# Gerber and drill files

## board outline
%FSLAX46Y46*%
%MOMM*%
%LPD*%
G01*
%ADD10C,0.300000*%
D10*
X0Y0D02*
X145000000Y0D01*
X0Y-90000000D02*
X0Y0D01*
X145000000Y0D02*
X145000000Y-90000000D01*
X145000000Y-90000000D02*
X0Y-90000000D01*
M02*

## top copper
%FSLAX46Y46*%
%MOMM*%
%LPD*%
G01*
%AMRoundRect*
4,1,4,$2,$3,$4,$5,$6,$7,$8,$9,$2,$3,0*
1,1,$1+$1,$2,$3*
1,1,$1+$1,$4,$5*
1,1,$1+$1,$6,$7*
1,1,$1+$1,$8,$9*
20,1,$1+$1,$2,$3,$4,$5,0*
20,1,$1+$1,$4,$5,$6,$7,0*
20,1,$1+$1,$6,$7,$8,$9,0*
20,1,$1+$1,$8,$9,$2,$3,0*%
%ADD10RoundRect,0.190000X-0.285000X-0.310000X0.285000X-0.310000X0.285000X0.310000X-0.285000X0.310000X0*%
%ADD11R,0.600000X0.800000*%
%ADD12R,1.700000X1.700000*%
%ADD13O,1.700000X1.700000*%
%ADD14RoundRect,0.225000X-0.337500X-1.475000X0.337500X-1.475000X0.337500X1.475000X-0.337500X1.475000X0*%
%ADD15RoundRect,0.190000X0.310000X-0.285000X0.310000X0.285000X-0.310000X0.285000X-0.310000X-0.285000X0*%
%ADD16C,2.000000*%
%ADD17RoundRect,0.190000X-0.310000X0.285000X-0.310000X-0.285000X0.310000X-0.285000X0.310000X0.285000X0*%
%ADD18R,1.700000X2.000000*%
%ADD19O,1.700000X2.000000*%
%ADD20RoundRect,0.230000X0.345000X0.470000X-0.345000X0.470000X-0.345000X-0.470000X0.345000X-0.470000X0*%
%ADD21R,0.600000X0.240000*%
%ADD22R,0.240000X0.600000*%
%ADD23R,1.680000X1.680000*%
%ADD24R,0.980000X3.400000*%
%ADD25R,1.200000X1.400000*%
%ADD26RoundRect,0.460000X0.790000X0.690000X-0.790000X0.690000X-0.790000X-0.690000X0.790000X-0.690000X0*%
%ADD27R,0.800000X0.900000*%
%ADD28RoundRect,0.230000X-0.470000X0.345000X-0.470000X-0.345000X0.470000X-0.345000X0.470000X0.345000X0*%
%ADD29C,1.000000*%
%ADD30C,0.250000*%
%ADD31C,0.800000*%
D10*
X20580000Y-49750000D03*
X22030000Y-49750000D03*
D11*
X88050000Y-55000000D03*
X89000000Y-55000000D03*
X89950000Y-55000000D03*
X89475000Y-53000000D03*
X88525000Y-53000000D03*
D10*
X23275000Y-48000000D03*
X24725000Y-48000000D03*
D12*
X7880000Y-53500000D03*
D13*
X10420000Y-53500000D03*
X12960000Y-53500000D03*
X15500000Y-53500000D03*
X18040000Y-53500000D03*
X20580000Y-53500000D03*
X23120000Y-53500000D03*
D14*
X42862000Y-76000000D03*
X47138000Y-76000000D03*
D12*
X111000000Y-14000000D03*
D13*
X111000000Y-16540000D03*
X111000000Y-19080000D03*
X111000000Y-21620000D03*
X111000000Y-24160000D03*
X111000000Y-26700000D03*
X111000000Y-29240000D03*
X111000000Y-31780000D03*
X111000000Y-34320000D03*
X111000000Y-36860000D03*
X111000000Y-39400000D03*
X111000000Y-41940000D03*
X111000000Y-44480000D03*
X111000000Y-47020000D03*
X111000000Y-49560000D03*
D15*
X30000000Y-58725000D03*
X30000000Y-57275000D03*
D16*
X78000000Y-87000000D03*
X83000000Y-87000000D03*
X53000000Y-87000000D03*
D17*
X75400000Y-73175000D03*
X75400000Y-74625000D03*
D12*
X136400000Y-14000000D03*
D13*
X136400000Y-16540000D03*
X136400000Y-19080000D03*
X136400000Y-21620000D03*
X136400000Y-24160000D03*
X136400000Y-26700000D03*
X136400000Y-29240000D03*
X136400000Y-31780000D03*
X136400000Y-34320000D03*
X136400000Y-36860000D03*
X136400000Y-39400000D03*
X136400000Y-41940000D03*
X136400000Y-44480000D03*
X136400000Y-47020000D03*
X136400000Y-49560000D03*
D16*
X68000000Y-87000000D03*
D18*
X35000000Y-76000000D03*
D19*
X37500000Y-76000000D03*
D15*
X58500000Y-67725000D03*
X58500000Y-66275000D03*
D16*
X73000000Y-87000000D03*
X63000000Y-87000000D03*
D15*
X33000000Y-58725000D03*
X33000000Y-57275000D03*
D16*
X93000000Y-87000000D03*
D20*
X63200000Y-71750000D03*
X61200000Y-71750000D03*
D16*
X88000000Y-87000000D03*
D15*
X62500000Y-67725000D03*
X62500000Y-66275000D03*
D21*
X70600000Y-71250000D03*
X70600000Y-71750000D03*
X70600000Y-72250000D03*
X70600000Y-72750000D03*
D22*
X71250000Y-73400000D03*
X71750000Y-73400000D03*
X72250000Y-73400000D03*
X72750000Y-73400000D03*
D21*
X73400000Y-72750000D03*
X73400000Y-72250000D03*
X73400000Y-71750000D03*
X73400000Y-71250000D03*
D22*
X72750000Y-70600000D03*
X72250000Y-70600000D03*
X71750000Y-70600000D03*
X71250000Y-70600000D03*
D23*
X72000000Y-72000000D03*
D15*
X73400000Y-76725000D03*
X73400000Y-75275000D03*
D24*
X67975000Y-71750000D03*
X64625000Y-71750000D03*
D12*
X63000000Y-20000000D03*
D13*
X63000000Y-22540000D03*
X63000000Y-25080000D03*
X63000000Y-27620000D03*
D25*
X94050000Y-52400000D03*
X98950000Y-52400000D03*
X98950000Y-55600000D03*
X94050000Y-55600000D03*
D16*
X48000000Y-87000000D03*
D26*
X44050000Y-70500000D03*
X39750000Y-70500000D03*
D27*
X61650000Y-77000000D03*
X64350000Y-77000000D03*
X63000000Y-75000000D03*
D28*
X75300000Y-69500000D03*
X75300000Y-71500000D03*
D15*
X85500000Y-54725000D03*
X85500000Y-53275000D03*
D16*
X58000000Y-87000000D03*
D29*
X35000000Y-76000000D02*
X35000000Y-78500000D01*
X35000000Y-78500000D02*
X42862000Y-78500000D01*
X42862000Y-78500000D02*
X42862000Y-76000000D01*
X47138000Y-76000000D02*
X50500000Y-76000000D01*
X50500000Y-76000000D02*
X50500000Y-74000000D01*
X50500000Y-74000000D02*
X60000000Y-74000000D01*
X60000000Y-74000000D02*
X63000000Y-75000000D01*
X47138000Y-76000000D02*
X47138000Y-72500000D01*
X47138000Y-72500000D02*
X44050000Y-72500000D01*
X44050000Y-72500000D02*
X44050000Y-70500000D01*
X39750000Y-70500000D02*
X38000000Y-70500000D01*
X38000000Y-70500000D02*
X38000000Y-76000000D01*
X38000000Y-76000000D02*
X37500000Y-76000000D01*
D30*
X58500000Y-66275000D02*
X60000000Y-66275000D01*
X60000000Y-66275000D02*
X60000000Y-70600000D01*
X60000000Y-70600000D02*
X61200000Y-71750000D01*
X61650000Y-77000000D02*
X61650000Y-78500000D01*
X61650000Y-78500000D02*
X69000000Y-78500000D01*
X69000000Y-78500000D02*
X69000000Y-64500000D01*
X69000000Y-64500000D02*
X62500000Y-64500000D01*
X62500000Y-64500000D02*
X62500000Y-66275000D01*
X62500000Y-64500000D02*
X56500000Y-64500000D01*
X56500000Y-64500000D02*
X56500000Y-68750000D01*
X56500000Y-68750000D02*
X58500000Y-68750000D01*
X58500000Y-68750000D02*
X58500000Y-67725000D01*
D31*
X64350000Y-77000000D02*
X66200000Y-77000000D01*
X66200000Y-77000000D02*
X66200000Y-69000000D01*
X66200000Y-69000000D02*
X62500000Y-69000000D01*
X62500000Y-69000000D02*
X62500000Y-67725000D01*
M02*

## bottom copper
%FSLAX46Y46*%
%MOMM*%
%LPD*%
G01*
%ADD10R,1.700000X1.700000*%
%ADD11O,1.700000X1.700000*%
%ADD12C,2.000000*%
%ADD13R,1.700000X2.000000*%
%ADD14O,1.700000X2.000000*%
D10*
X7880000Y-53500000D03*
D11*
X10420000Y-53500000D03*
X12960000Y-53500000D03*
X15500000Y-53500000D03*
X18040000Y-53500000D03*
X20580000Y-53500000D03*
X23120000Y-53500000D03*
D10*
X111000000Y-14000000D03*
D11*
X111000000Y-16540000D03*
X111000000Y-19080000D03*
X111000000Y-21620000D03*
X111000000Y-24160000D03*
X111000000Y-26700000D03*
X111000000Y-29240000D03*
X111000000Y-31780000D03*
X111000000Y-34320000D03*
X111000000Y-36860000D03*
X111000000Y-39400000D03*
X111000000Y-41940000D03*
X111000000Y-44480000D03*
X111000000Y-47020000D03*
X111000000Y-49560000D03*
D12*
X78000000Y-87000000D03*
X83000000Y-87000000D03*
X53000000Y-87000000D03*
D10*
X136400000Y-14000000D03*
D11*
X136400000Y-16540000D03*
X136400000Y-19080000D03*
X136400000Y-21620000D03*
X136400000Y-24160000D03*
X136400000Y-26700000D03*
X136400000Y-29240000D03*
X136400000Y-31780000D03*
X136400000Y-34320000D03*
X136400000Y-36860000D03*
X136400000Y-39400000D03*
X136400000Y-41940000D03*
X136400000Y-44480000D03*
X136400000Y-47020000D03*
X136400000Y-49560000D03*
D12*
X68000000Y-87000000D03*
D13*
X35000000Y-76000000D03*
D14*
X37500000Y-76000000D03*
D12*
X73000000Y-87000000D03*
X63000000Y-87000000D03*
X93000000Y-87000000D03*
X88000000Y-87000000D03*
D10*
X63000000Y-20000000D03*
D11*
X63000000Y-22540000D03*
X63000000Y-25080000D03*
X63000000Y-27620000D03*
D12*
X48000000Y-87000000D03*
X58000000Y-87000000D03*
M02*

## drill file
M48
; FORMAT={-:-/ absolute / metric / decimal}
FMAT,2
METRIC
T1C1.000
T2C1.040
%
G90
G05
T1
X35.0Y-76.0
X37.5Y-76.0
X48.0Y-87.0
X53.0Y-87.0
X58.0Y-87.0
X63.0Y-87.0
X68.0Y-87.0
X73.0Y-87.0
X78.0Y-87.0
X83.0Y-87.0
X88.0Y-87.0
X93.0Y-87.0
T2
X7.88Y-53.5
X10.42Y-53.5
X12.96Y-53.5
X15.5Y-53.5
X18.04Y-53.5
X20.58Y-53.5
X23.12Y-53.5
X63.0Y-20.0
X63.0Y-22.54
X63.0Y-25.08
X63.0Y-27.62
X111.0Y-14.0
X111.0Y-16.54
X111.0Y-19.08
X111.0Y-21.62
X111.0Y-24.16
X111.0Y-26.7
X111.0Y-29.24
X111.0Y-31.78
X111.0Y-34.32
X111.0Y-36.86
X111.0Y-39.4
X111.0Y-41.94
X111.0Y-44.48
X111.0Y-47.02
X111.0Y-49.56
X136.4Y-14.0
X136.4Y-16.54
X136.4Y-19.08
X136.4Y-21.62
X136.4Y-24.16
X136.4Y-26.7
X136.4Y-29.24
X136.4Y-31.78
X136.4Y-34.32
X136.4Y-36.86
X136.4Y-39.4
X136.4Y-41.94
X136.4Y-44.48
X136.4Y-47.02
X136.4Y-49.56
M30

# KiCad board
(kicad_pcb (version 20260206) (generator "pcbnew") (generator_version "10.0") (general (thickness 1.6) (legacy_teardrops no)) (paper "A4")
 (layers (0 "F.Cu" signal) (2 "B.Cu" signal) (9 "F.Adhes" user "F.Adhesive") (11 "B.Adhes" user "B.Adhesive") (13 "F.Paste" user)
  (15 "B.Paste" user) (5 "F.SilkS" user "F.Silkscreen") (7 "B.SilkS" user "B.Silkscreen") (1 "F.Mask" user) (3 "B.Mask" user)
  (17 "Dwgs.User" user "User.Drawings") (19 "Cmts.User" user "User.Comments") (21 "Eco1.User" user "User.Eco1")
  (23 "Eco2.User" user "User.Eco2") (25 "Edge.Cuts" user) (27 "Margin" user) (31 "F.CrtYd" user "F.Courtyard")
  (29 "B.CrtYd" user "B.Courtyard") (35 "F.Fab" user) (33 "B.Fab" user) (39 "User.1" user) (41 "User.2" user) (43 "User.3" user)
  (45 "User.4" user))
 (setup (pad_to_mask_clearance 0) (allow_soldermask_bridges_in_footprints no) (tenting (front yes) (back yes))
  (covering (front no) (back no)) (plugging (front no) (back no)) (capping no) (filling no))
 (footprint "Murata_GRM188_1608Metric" (layer "F.Cu") (at 21.305 49.75)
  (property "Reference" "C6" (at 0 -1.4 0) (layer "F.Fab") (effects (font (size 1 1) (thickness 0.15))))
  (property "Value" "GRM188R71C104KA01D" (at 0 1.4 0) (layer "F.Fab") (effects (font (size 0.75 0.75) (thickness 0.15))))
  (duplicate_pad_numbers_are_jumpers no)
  (pad "1" smd roundrect (at -0.725 0) (size 0.95 1) (layers "F.Cu" "F.Mask" "F.Paste") (roundrect_rratio 0.2) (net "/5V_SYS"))
  (pad "2" smd roundrect (at 0.725 0) (size 0.95 1) (layers "F.Cu" "F.Mask" "F.Paste") (roundrect_rratio 0.2) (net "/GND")))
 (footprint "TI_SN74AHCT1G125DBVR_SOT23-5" (layer "F.Cu") (at 89 54)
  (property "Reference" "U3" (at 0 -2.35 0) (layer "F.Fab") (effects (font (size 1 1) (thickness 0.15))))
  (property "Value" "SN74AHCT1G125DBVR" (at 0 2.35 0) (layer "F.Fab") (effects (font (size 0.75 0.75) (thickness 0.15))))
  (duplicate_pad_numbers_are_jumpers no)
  (pad "1" smd rect (at -0.95 1) (size 0.6 0.8) (layers "F.Cu" "F.Mask" "F.Paste") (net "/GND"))
  (pad "2" smd rect (at 0 1) (size 0.6 0.8) (layers "F.Cu" "F.Mask" "F.Paste") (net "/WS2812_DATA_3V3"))
  (pad "3" smd rect (at 0.95 1) (size 0.6 0.8) (layers "F.Cu" "F.Mask" "F.Paste") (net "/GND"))
  (pad "4" smd rect (at 0.475 -1) (size 0.6 0.8) (layers "F.Cu" "F.Mask" "F.Paste") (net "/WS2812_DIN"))
  (pad "5" smd rect (at -0.475 -1) (size 0.6 0.8) (layers "F.Cu" "F.Mask" "F.Paste") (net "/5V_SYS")))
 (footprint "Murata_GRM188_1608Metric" (layer "F.Cu") (at 24 48)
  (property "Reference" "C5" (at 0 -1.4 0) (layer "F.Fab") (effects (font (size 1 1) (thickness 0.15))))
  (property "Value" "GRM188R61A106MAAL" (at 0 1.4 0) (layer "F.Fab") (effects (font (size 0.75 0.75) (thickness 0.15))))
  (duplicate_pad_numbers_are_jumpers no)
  (pad "1" smd roundrect (at -0.725 0) (size 0.95 1) (layers "F.Cu" "F.Mask" "F.Paste") (roundrect_rratio 0.2) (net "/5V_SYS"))
  (pad "2" smd roundrect (at 0.725 0) (size 0.95 1) (layers "F.Cu" "F.Mask" "F.Paste") (roundrect_rratio 0.2) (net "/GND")))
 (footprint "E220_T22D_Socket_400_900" (layer "F.Cu") (at 5 52)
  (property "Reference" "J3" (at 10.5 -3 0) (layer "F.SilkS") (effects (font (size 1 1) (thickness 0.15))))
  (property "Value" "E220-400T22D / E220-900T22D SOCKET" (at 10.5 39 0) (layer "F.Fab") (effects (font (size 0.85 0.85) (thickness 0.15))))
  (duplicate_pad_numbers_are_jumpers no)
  (pad "1" thru_hole rect (at 2.88 1.5) (size 1.7 1.7) (drill 1.04) (layers "*.Cu" "*.Mask") (remove_unused_layers no) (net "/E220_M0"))
  (pad "2" thru_hole oval (at 5.42 1.5) (size 1.7 1.7) (drill 1.04) (layers "*.Cu" "*.Mask") (remove_unused_layers no) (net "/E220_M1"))
  (pad "3" thru_hole oval (at 7.96 1.5) (size 1.7 1.7) (drill 1.04) (layers "*.Cu" "*.Mask") (remove_unused_layers no) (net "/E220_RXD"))
  (pad "4" thru_hole oval (at 10.5 1.5) (size 1.7 1.7) (drill 1.04) (layers "*.Cu" "*.Mask") (remove_unused_layers no) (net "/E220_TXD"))
  (pad "5" thru_hole oval (at 13.04 1.5) (size 1.7 1.7) (drill 1.04) (layers "*.Cu" "*.Mask") (remove_unused_layers no) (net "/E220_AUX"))
  (pad "6" thru_hole oval (at 15.58 1.5) (size 1.7 1.7) (drill 1.04) (layers "*.Cu" "*.Mask") (remove_unused_layers no) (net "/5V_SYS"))
  (pad "7" thru_hole oval (at 18.12 1.5) (size 1.7 1.7) (drill 1.04) (layers "*.Cu" "*.Mask") (remove_unused_layers no) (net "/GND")))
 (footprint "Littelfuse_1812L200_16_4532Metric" (layer "F.Cu") (at 45 76)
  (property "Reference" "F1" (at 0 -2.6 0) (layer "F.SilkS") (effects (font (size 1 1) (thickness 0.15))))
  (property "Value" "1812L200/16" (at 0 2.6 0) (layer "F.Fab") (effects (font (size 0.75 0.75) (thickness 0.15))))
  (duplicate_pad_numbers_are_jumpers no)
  (pad "1" smd roundrect (at -2.138 0) (size 1.125 3.4) (layers "F.Cu" "F.Mask" "F.Paste") (roundrect_rratio 0.2) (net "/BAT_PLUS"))
  (pad "2" smd roundrect (at 2.138 0) (size 1.125 3.4) (layers "F.Cu" "F.Mask" "F.Paste") (roundrect_rratio 0.2) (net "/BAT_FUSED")))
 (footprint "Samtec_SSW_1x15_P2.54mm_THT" (layer "F.Cu") (at 111 14)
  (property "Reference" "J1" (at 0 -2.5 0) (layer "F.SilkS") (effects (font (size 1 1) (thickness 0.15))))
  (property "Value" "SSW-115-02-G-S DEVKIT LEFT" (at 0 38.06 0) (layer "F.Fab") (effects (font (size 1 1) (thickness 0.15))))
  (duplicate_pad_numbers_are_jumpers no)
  (pad "1" thru_hole rect (at 0 0) (size 1.7 1.7) (drill 1.04) (layers "*.Cu" "*.Mask") (remove_unused_layers no) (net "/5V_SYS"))
  (pad "2" thru_hole oval (at 0 2.54) (size 1.7 1.7) (drill 1.04) (layers "*.Cu" "*.Mask") (remove_unused_layers no) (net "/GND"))
  (pad "3" thru_hole oval (at 0 5.08) (size 1.7 1.7) (drill 1.04) (layers "*.Cu" "*.Mask") (remove_unused_layers no))
  (pad "4" thru_hole oval (at 0 7.62) (size 1.7 1.7) (drill 1.04) (layers "*.Cu" "*.Mask") (remove_unused_layers no))
  (pad "5" thru_hole oval (at 0 10.16) (size 1.7 1.7) (drill 1.04) (layers "*.Cu" "*.Mask") (remove_unused_layers no))
  (pad "6" thru_hole oval (at 0 12.7) (size 1.7 1.7) (drill 1.04) (layers "*.Cu" "*.Mask") (remove_unused_layers no) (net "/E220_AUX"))
  (pad "7" thru_hole oval (at 0 15.24) (size 1.7 1.7) (drill 1.04) (layers "*.Cu" "*.Mask") (remove_unused_layers no) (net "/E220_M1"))
  (pad "8" thru_hole oval (at 0 17.78) (size 1.7 1.7) (drill 1.04) (layers "*.Cu" "*.Mask") (remove_unused_layers no) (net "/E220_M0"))
  (pad "9" thru_hole oval (at 0 20.32) (size 1.7 1.7) (drill 1.04) (layers "*.Cu" "*.Mask") (remove_unused_layers no))
  (pad "10" thru_hole oval (at 0 22.86) (size 1.7 1.7) (drill 1.04) (layers "*.Cu" "*.Mask") (remove_unused_layers no))
  (pad "11" thru_hole oval (at 0 25.4) (size 1.7 1.7) (drill 1.04) (layers "*.Cu" "*.Mask") (remove_unused_layers no))
  (pad "12" thru_hole oval (at 0 27.94) (size 1.7 1.7) (drill 1.04) (layers "*.Cu" "*.Mask") (remove_unused_layers no))
  (pad "13" thru_hole oval (at 0 30.48) (size 1.7 1.7) (drill 1.04) (layers "*.Cu" "*.Mask") (remove_unused_layers no))
  (pad "14" thru_hole oval (at 0 33.02) (size 1.7 1.7) (drill 1.04) (layers "*.Cu" "*.Mask") (remove_unused_layers no))
  (pad "15" thru_hole oval (at 0 35.56) (size 1.7 1.7) (drill 1.04) (layers "*.Cu" "*.Mask") (remove_unused_layers no)))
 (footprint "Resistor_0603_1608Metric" (layer "F.Cu") (at 30 58 90)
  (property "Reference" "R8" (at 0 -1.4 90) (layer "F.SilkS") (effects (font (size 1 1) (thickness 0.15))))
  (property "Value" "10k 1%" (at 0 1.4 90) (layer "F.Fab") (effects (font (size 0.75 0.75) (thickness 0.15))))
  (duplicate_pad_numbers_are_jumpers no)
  (pad "1" smd roundrect (at -0.725 0 90) (size 0.95 1) (layers "F.Cu" "F.Mask" "F.Paste") (roundrect_rratio 0.2) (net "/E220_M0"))
  (pad "2" smd roundrect (at 0.725 0 90) (size 0.95 1) (layers "F.Cu" "F.Mask" "F.Paste") (roundrect_rratio 0.2) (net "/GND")))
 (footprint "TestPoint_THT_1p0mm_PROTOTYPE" (layer "F.Cu") (at 78 87)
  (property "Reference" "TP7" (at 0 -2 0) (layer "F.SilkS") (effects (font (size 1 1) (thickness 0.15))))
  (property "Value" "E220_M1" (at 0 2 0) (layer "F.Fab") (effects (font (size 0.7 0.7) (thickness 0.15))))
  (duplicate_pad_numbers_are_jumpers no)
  (pad "1" thru_hole circle (at 0 0) (size 2 2) (drill 1) (layers "*.Cu" "*.Mask") (remove_unused_layers no) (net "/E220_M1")))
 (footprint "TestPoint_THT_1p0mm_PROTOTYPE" (layer "F.Cu") (at 83 87)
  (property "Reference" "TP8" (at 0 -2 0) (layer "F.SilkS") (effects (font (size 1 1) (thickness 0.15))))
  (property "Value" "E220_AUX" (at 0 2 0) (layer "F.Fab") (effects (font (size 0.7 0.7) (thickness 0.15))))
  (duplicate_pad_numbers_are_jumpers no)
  (pad "1" thru_hole circle (at 0 0) (size 2 2) (drill 1) (layers "*.Cu" "*.Mask") (remove_unused_layers no) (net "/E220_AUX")))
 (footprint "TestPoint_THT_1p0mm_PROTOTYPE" (layer "F.Cu") (at 53 87)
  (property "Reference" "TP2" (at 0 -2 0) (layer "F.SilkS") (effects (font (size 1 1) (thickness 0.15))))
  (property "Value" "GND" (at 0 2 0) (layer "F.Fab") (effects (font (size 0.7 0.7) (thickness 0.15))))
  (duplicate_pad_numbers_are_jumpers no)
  (pad "1" thru_hole circle (at 0 0) (size 2 2) (drill 1) (layers "*.Cu" "*.Mask") (remove_unused_layers no) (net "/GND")))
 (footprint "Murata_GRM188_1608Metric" (layer "F.Cu") (at 75.4 73.9 -90)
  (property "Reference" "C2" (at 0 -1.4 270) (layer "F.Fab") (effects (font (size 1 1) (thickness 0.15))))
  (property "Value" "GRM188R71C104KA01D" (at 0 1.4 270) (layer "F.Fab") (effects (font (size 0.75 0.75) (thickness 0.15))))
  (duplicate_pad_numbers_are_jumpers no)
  (pad "1" smd roundrect (at -0.725 0 270) (size 0.95 1) (layers "F.Cu" "F.Mask" "F.Paste") (roundrect_rratio 0.2) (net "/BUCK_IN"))
  (pad "2" smd roundrect (at 0.725 0 270) (size 0.95 1) (layers "F.Cu" "F.Mask" "F.Paste") (roundrect_rratio 0.2) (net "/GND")))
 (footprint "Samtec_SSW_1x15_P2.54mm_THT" (layer "F.Cu") (at 136.4 14)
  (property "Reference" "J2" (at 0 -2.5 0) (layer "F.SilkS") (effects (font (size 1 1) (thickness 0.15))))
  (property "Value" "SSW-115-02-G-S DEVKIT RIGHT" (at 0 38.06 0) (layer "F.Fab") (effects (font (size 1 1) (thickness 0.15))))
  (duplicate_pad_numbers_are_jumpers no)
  (pad "1" thru_hole rect (at 0 0) (size 1.7 1.7) (drill 1.04) (layers "*.Cu" "*.Mask") (remove_unused_layers no) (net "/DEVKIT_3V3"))
  (pad "2" thru_hole oval (at 0 2.54) (size 1.7 1.7) (drill 1.04) (layers "*.Cu" "*.Mask") (remove_unused_layers no) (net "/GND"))
  (pad "3" thru_hole oval (at 0 5.08) (size 1.7 1.7) (drill 1.04) (layers "*.Cu" "*.Mask") (remove_unused_layers no))
  (pad "4" thru_hole oval (at 0 7.62) (size 1.7 1.7) (drill 1.04) (layers "*.Cu" "*.Mask") (remove_unused_layers no))
  (pad "5" thru_hole oval (at 0 10.16) (size 1.7 1.7) (drill 1.04) (layers "*.Cu" "*.Mask") (remove_unused_layers no)
   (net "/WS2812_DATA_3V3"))
  (pad "6" thru_hole oval (at 0 12.7) (size 1.7 1.7) (drill 1.04) (layers "*.Cu" "*.Mask") (remove_unused_layers no) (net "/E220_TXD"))
  (pad "7" thru_hole oval (at 0 15.24) (size 1.7 1.7) (drill 1.04) (layers "*.Cu" "*.Mask") (remove_unused_layers no) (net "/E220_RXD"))
  (pad "8" thru_hole oval (at 0 17.78) (size 1.7 1.7) (drill 1.04) (layers "*.Cu" "*.Mask") (remove_unused_layers no))
  (pad "9" thru_hole oval (at 0 20.32) (size 1.7 1.7) (drill 1.04) (layers "*.Cu" "*.Mask") (remove_unused_layers no))
  (pad "10" thru_hole oval (at 0 22.86) (size 1.7 1.7) (drill 1.04) (layers "*.Cu" "*.Mask") (remove_unused_layers no))
  (pad "11" thru_hole oval (at 0 25.4) (size 1.7 1.7) (drill 1.04) (layers "*.Cu" "*.Mask") (remove_unused_layers no) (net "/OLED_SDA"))
  (pad "12" thru_hole oval (at 0 27.94) (size 1.7 1.7) (drill 1.04) (layers "*.Cu" "*.Mask") (remove_unused_layers no))
  (pad "13" thru_hole oval (at 0 30.48) (size 1.7 1.7) (drill 1.04) (layers "*.Cu" "*.Mask") (remove_unused_layers no))
  (pad "14" thru_hole oval (at 0 33.02) (size 1.7 1.7) (drill 1.04) (layers "*.Cu" "*.Mask") (remove_unused_layers no) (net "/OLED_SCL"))
  (pad "15" thru_hole oval (at 0 35.56) (size 1.7 1.7) (drill 1.04) (layers "*.Cu" "*.Mask") (remove_unused_layers no)))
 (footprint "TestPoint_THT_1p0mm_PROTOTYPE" (layer "F.Cu") (at 68 87)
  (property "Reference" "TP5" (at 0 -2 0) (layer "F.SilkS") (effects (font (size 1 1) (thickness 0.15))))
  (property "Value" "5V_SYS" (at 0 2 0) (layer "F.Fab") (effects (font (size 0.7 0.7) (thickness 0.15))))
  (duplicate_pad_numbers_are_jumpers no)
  (pad "1" thru_hole circle (at 0 0) (size 2 2) (drill 1) (layers "*.Cu" "*.Mask") (remove_unused_layers no) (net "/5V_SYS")))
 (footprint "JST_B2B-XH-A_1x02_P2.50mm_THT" (layer "F.Cu") (at 35 76)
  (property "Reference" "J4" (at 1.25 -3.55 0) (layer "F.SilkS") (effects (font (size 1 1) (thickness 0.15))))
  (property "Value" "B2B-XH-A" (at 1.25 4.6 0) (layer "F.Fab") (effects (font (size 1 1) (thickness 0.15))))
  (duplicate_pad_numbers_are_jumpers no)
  (pad "1" thru_hole rect (at 0 0) (size 1.7 2) (drill 1) (layers "*.Cu" "*.Mask") (remove_unused_layers no) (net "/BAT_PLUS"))
  (pad "2" thru_hole oval (at 2.5 0) (size 1.7 2) (drill 1) (layers "*.Cu" "*.Mask") (remove_unused_layers no) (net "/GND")))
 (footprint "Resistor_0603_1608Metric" (layer "F.Cu") (at 58.5 67 90)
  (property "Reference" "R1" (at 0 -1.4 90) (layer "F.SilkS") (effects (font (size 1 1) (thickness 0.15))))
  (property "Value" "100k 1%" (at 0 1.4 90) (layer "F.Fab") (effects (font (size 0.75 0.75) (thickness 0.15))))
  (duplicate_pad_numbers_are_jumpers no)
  (pad "1" smd roundrect (at -0.725 0 90) (size 0.95 1) (layers "F.Cu" "F.Mask" "F.Paste") (roundrect_rratio 0.2) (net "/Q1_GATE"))
  (pad "2" smd roundrect (at 0.725 0 90) (size 0.95 1) (layers "F.Cu" "F.Mask" "F.Paste") (roundrect_rratio 0.2) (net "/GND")))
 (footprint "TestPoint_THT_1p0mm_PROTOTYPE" (layer "F.Cu") (at 73 87)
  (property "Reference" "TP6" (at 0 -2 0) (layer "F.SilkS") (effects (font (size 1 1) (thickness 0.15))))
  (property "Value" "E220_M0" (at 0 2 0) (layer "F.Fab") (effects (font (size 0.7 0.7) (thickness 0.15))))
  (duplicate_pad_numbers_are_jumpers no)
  (pad "1" thru_hole circle (at 0 0) (size 2 2) (drill 1) (layers "*.Cu" "*.Mask") (remove_unused_layers no) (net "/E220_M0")))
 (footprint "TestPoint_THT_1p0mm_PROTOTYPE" (layer "F.Cu") (at 63 87)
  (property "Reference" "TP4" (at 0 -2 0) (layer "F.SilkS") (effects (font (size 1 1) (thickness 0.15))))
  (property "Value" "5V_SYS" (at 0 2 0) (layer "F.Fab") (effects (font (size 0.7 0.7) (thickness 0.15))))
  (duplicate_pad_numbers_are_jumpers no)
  (pad "1" thru_hole circle (at 0 0) (size 2 2) (drill 1) (layers "*.Cu" "*.Mask") (remove_unused_layers no) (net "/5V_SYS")))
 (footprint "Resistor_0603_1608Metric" (layer "F.Cu") (at 33 58 90)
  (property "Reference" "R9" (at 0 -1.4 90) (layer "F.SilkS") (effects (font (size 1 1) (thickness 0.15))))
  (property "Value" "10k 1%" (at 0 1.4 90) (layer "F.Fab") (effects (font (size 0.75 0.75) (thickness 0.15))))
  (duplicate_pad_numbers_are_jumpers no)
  (pad "1" smd roundrect (at -0.725 0 90) (size 0.95 1) (layers "F.Cu" "F.Mask" "F.Paste") (roundrect_rratio 0.2) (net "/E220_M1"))
  (pad "2" smd roundrect (at 0.725 0 90) (size 0.95 1) (layers "F.Cu" "F.Mask" "F.Paste") (roundrect_rratio 0.2) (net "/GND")))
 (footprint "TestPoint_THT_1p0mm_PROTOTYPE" (layer "F.Cu") (at 93 87)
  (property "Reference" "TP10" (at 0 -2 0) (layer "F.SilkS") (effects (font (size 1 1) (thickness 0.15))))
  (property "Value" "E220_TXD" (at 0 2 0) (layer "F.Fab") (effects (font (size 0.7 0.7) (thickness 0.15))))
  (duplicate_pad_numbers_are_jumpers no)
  (pad "1" thru_hole circle (at 0 0) (size 2 2) (drill 1) (layers "*.Cu" "*.Mask") (remove_unused_layers no) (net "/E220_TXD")))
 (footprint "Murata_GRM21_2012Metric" (layer "F.Cu") (at 62.2 71.75 180)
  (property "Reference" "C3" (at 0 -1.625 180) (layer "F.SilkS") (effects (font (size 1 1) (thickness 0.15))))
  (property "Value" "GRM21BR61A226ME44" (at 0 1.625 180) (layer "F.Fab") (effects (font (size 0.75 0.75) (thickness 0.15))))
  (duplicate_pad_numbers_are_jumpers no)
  (pad "1" smd roundrect (at -1 0 180) (size 1.15 1.4) (layers "F.Cu" "F.Mask" "F.Paste") (roundrect_rratio 0.2) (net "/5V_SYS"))
  (pad "2" smd roundrect (at 1 0 180) (size 1.15 1.4) (layers "F.Cu" "F.Mask" "F.Paste") (roundrect_rratio 0.2) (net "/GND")))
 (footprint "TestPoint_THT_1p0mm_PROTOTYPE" (layer "F.Cu") (at 88 87)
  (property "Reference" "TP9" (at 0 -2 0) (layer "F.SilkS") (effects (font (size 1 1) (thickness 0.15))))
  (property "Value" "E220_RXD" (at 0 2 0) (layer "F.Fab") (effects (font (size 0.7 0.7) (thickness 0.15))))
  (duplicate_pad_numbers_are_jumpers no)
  (pad "1" thru_hole circle (at 0 0) (size 2 2) (drill 1) (layers "*.Cu" "*.Mask") (remove_unused_layers no) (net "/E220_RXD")))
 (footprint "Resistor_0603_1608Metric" (layer "F.Cu") (at 62.5 67 90)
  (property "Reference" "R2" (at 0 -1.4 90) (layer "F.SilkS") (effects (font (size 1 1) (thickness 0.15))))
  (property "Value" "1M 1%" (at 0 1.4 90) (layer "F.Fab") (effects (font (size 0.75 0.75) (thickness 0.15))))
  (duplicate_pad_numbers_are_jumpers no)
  (pad "1" smd roundrect (at -0.725 0 90) (size 0.95 1) (layers "F.Cu" "F.Mask" "F.Paste") (roundrect_rratio 0.2) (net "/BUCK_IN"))
  (pad "2" smd roundrect (at 0.725 0 90) (size 0.95 1) (layers "F.Cu" "F.Mask" "F.Paste") (roundrect_rratio 0.2) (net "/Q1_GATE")))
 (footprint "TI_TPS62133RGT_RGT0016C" (layer "F.Cu") (at 72 72)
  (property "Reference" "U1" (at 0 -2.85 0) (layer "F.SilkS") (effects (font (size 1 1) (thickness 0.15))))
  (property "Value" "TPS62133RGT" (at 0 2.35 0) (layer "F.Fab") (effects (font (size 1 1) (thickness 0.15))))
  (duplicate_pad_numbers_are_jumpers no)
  (pad "" smd rect (at 0 0) (size 1.55 1.55) (layers "F.Paste"))
  (pad "1" smd rect (at -1.4 -0.75) (size 0.6 0.24) (layers "F.Cu" "F.Mask" "F.Paste") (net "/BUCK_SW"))
  (pad "2" smd rect (at -1.4 -0.25) (size 0.6 0.24) (layers "F.Cu" "F.Mask" "F.Paste") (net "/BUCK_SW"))
  (pad "3" smd rect (at -1.4 0.25) (size 0.6 0.24) (layers "F.Cu" "F.Mask" "F.Paste") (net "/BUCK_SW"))
  (pad "4" smd rect (at -1.4 0.75) (size 0.6 0.24) (layers "F.Cu" "F.Mask" "F.Paste"))
  (pad "5" smd rect (at -0.75 1.4) (size 0.24 0.6) (layers "F.Cu" "F.Mask" "F.Paste") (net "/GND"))
  (pad "6" smd rect (at -0.25 1.4) (size 0.24 0.6) (layers "F.Cu" "F.Mask" "F.Paste") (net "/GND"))
  (pad "7" smd rect (at 0.25 1.4) (size 0.24 0.6) (layers "F.Cu" "F.Mask" "F.Paste") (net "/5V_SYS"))
  (pad "8" smd rect (at 0.75 1.4) (size 0.24 0.6) (layers "F.Cu" "F.Mask" "F.Paste") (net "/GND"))
  (pad "9" smd rect (at 1.4 0.75) (size 0.6 0.24) (layers "F.Cu" "F.Mask" "F.Paste") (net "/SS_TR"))
  (pad "10" smd rect (at 1.4 0.25) (size 0.6 0.24) (layers "F.Cu" "F.Mask" "F.Paste") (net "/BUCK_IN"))
  (pad "11" smd rect (at 1.4 -0.25) (size 0.6 0.24) (layers "F.Cu" "F.Mask" "F.Paste") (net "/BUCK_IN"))
  (pad "12" smd rect (at 1.4 -0.75) (size 0.6 0.24) (layers "F.Cu" "F.Mask" "F.Paste") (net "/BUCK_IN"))
  (pad "13" smd rect (at 0.75 -1.4) (size 0.24 0.6) (layers "F.Cu" "F.Mask" "F.Paste") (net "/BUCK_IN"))
  (pad "14" smd rect (at 0.25 -1.4) (size 0.24 0.6) (layers "F.Cu" "F.Mask" "F.Paste") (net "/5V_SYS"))
  (pad "15" smd rect (at -0.25 -1.4) (size 0.24 0.6) (layers "F.Cu" "F.Mask" "F.Paste") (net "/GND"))
  (pad "16" smd rect (at -0.75 -1.4) (size 0.24 0.6) (layers "F.Cu" "F.Mask" "F.Paste") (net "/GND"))
  (pad "EP" smd rect (at 0 0) (size 1.68 1.68) (layers "F.Cu" "F.Mask") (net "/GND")))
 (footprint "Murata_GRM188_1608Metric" (layer "F.Cu") (at 73.4 76 90)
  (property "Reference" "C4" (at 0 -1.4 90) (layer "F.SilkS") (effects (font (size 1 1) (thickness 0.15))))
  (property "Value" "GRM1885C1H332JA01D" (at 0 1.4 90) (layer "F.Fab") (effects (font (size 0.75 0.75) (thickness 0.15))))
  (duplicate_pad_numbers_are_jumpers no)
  (pad "1" smd roundrect (at -0.725 0 90) (size 0.95 1) (layers "F.Cu" "F.Mask" "F.Paste") (roundrect_rratio 0.2) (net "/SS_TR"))
  (pad "2" smd roundrect (at 0.725 0 90) (size 0.95 1) (layers "F.Cu" "F.Mask" "F.Paste") (roundrect_rratio 0.2) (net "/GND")))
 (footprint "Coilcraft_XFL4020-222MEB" (layer "F.Cu") (at 66.3 71.75 180)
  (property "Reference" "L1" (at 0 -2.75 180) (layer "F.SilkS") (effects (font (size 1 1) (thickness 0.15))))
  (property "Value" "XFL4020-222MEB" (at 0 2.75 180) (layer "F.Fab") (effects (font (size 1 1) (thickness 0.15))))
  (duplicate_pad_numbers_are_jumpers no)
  (pad "1" smd rect (at -1.675 0 180) (size 0.98 3.4) (layers "F.Cu" "F.Mask" "F.Paste") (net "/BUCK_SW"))
  (pad "2" smd rect (at 1.675 0 180) (size 0.98 3.4) (layers "F.Cu" "F.Mask" "F.Paste") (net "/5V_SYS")))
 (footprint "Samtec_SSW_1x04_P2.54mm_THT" (layer "F.Cu") (at 63 20)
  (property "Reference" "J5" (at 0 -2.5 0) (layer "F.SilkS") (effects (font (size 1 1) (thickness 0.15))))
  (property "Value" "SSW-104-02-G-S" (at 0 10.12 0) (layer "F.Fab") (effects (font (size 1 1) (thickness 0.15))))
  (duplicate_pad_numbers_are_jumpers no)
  (pad "1" thru_hole rect (at 0 0) (size 1.7 1.7) (drill 1.04) (layers "*.Cu" "*.Mask") (remove_unused_layers no) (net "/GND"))
  (pad "2" thru_hole oval (at 0 2.54) (size 1.7 1.7) (drill 1.04) (layers "*.Cu" "*.Mask") (remove_unused_layers no) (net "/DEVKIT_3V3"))
  (pad "3" thru_hole oval (at 0 5.08) (size 1.7 1.7) (drill 1.04) (layers "*.Cu" "*.Mask") (remove_unused_layers no) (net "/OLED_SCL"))
  (pad "4" thru_hole oval (at 0 7.62) (size 1.7 1.7) (drill 1.04) (layers "*.Cu" "*.Mask") (remove_unused_layers no) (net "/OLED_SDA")))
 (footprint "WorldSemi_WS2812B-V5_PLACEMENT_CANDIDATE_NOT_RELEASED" (layer "F.Cu") (at 96.5 54)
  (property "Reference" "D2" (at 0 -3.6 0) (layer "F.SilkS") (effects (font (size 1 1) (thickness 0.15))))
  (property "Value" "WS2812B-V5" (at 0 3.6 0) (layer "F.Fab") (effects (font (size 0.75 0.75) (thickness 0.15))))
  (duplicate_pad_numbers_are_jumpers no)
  (pad "1" smd rect (at -2.45 -1.6) (size 1.2 1.4) (layers "F.Cu" "F.Mask" "F.Paste") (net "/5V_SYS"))
  (pad "2" smd rect (at 2.45 -1.6) (size 1.2 1.4) (layers "F.Cu" "F.Mask" "F.Paste"))
  (pad "3" smd rect (at 2.45 1.6) (size 1.2 1.4) (layers "F.Cu" "F.Mask" "F.Paste") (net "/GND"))
  (pad "4" smd rect (at -2.45 1.6) (size 1.2 1.4) (layers "F.Cu" "F.Mask" "F.Paste") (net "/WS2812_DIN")))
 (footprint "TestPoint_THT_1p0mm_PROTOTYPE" (layer "F.Cu") (at 48 87)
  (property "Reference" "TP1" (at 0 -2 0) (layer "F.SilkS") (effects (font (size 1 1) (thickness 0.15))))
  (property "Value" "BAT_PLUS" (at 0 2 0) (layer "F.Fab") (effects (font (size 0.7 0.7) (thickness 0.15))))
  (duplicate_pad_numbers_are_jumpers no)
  (pad "1" thru_hole circle (at 0 0) (size 2 2) (drill 1) (layers "*.Cu" "*.Mask") (remove_unused_layers no) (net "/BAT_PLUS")))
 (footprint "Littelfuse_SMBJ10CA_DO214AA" (layer "F.Cu") (at 41.9 70.5 180)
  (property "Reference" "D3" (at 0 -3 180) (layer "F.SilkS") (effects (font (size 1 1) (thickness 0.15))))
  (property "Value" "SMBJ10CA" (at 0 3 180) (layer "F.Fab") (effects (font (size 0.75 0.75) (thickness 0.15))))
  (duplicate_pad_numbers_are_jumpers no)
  (pad "1" smd roundrect (at -2.15 0 180) (size 2.5 2.3) (layers "F.Cu" "F.Mask" "F.Paste") (roundrect_rratio 0.2) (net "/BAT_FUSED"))
  (pad "2" smd roundrect (at 2.15 0 180) (size 2.5 2.3) (layers "F.Cu" "F.Mask" "F.Paste") (roundrect_rratio 0.2) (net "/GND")))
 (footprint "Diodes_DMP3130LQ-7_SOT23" (layer "F.Cu") (at 63 76)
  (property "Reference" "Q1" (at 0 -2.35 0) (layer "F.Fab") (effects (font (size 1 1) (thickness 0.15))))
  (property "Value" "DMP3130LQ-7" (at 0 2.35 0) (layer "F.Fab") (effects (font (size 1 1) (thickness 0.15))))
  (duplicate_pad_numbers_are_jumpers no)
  (pad "1" smd rect (at -1.35 1) (size 0.8 0.9) (layers "F.Cu" "F.Mask" "F.Paste") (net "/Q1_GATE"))
  (pad "2" smd rect (at 1.35 1) (size 0.8 0.9) (layers "F.Cu" "F.Mask" "F.Paste") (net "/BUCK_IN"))
  (pad "3" smd rect (at 0 -1) (size 0.8 0.9) (layers "F.Cu" "F.Mask" "F.Paste") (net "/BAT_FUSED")))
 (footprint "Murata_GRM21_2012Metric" (layer "F.Cu") (at 75.3 70.5 -90)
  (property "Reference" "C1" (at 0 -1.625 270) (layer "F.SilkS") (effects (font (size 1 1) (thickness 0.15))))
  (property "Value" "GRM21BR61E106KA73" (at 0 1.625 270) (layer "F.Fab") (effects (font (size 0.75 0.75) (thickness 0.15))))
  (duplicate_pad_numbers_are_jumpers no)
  (pad "1" smd roundrect (at -1 0 270) (size 1.15 1.4) (layers "F.Cu" "F.Mask" "F.Paste") (roundrect_rratio 0.2) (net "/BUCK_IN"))
  (pad "2" smd roundrect (at 1 0 270) (size 1.15 1.4) (layers "F.Cu" "F.Mask" "F.Paste") (roundrect_rratio 0.2) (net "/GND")))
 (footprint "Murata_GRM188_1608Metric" (layer "F.Cu") (at 85.5 54 90)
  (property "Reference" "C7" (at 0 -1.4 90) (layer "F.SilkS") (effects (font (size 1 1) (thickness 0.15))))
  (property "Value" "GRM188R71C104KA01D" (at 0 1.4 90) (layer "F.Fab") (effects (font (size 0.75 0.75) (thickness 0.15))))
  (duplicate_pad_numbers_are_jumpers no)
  (pad "1" smd roundrect (at -0.725 0 90) (size 0.95 1) (layers "F.Cu" "F.Mask" "F.Paste") (roundrect_rratio 0.2) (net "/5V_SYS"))
  (pad "2" smd roundrect (at 0.725 0 90) (size 0.95 1) (layers "F.Cu" "F.Mask" "F.Paste") (roundrect_rratio 0.2) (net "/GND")))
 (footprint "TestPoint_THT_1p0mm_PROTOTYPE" (layer "F.Cu") (at 58 87)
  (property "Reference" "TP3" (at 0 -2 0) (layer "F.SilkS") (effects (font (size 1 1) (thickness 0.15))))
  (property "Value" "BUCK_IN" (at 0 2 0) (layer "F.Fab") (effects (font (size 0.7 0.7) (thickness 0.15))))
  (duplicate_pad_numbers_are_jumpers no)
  (pad "1" thru_hole circle (at 0 0) (size 2 2) (drill 1) (layers "*.Cu" "*.Mask") (remove_unused_layers no) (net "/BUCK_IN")))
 (gr_line (start 0 0) (end 145 0) (stroke (width 0.3) (type default)) (layer "Edge.Cuts"))
 (gr_line (start 0 90) (end 0 0) (stroke (width 0.3) (type default)) (layer "Edge.Cuts"))
 (gr_line (start 145 0) (end 145 90) (stroke (width 0.3) (type default)) (layer "Edge.Cuts"))
 (gr_line (start 145 90) (end 0 90) (stroke (width 0.3) (type default)) (layer "Edge.Cuts"))
 (segment (start 35 76) (end 35 78.5) (width 1) (layer "F.Cu") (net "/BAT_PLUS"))
 (segment (start 35 78.5) (end 42.862 78.5) (width 1) (layer "F.Cu") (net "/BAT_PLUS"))
 (segment (start 42.862 78.5) (end 42.862 76) (width 1) (layer "F.Cu") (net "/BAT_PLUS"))
 (segment (start 47.138 76) (end 50.5 76) (width 1) (layer "F.Cu") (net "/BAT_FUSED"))
 (segment (start 50.5 76) (end 50.5 74) (width 1) (layer "F.Cu") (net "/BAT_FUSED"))
 (segment (start 50.5 74) (end 60 74) (width 1) (layer "F.Cu") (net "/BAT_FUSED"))
 (segment (start 60 74) (end 63 75) (width 1) (layer "F.Cu") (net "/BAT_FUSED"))
 (segment (start 47.138 76) (end 47.138 72.5) (width 1) (layer "F.Cu") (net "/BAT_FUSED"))
 (segment (start 47.138 72.5) (end 44.05 72.5) (width 1) (layer "F.Cu") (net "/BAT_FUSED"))
 (segment (start 44.05 72.5) (end 44.05 70.5) (width 1) (layer "F.Cu") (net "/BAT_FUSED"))
 (segment (start 39.75 70.5) (end 38 70.5) (width 1) (layer "F.Cu") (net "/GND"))
 (segment (start 38 70.5) (end 38 76) (width 1) (layer "F.Cu") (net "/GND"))
 (segment (start 38 76) (end 37.5 76) (width 1) (layer "F.Cu") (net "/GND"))
 (segment (start 58.5 66.275) (end 60 66.275) (width 0.25) (layer "F.Cu") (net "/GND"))
 (segment (start 60 66.275) (end 60 70.6) (width 0.25) (layer "F.Cu") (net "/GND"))
 (segment (start 60 70.6) (end 61.2 71.75) (width 0.25) (layer "F.Cu") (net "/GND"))
 (segment (start 61.65 77) (end 61.65 78.5) (width 0.25) (layer "F.Cu") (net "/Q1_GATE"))
 (segment (start 61.65 78.5) (end 69 78.5) (width 0.25) (layer "F.Cu") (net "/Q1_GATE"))
 (segment (start 69 78.5) (end 69 64.5) (width 0.25) (layer "F.Cu") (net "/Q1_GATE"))
 (segment (start 69 64.5) (end 62.5 64.5) (width 0.25) (layer "F.Cu") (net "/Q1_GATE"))
 (segment (start 62.5 64.5) (end 62.5 66.275) (width 0.25) (layer "F.Cu") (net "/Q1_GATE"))
 (segment (start 62.5 64.5) (end 56.5 64.5) (width 0.25) (layer "F.Cu") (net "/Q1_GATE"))
 (segment (start 56.5 64.5) (end 56.5 68.75) (width 0.25) (layer "F.Cu") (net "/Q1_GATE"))
 (segment (start 56.5 68.75) (end 58.5 68.75) (width 0.25) (layer "F.Cu") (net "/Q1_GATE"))
 (segment (start 58.5 68.75) (end 58.5 67.725) (width 0.25) (layer "F.Cu") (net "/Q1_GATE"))
 (segment (start 64.35 77) (end 66.2 77) (width 0.8) (layer "F.Cu") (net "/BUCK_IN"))
 (segment (start 66.2 77) (end 66.2 69) (width 0.8) (layer "F.Cu") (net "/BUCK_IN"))
 (segment (start 66.2 69) (end 62.5 69) (width 0.8) (layer "F.Cu") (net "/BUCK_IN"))
 (segment (start 62.5 69) (end 62.5 67.725) (width 0.8) (layer "F.Cu") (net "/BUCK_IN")))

